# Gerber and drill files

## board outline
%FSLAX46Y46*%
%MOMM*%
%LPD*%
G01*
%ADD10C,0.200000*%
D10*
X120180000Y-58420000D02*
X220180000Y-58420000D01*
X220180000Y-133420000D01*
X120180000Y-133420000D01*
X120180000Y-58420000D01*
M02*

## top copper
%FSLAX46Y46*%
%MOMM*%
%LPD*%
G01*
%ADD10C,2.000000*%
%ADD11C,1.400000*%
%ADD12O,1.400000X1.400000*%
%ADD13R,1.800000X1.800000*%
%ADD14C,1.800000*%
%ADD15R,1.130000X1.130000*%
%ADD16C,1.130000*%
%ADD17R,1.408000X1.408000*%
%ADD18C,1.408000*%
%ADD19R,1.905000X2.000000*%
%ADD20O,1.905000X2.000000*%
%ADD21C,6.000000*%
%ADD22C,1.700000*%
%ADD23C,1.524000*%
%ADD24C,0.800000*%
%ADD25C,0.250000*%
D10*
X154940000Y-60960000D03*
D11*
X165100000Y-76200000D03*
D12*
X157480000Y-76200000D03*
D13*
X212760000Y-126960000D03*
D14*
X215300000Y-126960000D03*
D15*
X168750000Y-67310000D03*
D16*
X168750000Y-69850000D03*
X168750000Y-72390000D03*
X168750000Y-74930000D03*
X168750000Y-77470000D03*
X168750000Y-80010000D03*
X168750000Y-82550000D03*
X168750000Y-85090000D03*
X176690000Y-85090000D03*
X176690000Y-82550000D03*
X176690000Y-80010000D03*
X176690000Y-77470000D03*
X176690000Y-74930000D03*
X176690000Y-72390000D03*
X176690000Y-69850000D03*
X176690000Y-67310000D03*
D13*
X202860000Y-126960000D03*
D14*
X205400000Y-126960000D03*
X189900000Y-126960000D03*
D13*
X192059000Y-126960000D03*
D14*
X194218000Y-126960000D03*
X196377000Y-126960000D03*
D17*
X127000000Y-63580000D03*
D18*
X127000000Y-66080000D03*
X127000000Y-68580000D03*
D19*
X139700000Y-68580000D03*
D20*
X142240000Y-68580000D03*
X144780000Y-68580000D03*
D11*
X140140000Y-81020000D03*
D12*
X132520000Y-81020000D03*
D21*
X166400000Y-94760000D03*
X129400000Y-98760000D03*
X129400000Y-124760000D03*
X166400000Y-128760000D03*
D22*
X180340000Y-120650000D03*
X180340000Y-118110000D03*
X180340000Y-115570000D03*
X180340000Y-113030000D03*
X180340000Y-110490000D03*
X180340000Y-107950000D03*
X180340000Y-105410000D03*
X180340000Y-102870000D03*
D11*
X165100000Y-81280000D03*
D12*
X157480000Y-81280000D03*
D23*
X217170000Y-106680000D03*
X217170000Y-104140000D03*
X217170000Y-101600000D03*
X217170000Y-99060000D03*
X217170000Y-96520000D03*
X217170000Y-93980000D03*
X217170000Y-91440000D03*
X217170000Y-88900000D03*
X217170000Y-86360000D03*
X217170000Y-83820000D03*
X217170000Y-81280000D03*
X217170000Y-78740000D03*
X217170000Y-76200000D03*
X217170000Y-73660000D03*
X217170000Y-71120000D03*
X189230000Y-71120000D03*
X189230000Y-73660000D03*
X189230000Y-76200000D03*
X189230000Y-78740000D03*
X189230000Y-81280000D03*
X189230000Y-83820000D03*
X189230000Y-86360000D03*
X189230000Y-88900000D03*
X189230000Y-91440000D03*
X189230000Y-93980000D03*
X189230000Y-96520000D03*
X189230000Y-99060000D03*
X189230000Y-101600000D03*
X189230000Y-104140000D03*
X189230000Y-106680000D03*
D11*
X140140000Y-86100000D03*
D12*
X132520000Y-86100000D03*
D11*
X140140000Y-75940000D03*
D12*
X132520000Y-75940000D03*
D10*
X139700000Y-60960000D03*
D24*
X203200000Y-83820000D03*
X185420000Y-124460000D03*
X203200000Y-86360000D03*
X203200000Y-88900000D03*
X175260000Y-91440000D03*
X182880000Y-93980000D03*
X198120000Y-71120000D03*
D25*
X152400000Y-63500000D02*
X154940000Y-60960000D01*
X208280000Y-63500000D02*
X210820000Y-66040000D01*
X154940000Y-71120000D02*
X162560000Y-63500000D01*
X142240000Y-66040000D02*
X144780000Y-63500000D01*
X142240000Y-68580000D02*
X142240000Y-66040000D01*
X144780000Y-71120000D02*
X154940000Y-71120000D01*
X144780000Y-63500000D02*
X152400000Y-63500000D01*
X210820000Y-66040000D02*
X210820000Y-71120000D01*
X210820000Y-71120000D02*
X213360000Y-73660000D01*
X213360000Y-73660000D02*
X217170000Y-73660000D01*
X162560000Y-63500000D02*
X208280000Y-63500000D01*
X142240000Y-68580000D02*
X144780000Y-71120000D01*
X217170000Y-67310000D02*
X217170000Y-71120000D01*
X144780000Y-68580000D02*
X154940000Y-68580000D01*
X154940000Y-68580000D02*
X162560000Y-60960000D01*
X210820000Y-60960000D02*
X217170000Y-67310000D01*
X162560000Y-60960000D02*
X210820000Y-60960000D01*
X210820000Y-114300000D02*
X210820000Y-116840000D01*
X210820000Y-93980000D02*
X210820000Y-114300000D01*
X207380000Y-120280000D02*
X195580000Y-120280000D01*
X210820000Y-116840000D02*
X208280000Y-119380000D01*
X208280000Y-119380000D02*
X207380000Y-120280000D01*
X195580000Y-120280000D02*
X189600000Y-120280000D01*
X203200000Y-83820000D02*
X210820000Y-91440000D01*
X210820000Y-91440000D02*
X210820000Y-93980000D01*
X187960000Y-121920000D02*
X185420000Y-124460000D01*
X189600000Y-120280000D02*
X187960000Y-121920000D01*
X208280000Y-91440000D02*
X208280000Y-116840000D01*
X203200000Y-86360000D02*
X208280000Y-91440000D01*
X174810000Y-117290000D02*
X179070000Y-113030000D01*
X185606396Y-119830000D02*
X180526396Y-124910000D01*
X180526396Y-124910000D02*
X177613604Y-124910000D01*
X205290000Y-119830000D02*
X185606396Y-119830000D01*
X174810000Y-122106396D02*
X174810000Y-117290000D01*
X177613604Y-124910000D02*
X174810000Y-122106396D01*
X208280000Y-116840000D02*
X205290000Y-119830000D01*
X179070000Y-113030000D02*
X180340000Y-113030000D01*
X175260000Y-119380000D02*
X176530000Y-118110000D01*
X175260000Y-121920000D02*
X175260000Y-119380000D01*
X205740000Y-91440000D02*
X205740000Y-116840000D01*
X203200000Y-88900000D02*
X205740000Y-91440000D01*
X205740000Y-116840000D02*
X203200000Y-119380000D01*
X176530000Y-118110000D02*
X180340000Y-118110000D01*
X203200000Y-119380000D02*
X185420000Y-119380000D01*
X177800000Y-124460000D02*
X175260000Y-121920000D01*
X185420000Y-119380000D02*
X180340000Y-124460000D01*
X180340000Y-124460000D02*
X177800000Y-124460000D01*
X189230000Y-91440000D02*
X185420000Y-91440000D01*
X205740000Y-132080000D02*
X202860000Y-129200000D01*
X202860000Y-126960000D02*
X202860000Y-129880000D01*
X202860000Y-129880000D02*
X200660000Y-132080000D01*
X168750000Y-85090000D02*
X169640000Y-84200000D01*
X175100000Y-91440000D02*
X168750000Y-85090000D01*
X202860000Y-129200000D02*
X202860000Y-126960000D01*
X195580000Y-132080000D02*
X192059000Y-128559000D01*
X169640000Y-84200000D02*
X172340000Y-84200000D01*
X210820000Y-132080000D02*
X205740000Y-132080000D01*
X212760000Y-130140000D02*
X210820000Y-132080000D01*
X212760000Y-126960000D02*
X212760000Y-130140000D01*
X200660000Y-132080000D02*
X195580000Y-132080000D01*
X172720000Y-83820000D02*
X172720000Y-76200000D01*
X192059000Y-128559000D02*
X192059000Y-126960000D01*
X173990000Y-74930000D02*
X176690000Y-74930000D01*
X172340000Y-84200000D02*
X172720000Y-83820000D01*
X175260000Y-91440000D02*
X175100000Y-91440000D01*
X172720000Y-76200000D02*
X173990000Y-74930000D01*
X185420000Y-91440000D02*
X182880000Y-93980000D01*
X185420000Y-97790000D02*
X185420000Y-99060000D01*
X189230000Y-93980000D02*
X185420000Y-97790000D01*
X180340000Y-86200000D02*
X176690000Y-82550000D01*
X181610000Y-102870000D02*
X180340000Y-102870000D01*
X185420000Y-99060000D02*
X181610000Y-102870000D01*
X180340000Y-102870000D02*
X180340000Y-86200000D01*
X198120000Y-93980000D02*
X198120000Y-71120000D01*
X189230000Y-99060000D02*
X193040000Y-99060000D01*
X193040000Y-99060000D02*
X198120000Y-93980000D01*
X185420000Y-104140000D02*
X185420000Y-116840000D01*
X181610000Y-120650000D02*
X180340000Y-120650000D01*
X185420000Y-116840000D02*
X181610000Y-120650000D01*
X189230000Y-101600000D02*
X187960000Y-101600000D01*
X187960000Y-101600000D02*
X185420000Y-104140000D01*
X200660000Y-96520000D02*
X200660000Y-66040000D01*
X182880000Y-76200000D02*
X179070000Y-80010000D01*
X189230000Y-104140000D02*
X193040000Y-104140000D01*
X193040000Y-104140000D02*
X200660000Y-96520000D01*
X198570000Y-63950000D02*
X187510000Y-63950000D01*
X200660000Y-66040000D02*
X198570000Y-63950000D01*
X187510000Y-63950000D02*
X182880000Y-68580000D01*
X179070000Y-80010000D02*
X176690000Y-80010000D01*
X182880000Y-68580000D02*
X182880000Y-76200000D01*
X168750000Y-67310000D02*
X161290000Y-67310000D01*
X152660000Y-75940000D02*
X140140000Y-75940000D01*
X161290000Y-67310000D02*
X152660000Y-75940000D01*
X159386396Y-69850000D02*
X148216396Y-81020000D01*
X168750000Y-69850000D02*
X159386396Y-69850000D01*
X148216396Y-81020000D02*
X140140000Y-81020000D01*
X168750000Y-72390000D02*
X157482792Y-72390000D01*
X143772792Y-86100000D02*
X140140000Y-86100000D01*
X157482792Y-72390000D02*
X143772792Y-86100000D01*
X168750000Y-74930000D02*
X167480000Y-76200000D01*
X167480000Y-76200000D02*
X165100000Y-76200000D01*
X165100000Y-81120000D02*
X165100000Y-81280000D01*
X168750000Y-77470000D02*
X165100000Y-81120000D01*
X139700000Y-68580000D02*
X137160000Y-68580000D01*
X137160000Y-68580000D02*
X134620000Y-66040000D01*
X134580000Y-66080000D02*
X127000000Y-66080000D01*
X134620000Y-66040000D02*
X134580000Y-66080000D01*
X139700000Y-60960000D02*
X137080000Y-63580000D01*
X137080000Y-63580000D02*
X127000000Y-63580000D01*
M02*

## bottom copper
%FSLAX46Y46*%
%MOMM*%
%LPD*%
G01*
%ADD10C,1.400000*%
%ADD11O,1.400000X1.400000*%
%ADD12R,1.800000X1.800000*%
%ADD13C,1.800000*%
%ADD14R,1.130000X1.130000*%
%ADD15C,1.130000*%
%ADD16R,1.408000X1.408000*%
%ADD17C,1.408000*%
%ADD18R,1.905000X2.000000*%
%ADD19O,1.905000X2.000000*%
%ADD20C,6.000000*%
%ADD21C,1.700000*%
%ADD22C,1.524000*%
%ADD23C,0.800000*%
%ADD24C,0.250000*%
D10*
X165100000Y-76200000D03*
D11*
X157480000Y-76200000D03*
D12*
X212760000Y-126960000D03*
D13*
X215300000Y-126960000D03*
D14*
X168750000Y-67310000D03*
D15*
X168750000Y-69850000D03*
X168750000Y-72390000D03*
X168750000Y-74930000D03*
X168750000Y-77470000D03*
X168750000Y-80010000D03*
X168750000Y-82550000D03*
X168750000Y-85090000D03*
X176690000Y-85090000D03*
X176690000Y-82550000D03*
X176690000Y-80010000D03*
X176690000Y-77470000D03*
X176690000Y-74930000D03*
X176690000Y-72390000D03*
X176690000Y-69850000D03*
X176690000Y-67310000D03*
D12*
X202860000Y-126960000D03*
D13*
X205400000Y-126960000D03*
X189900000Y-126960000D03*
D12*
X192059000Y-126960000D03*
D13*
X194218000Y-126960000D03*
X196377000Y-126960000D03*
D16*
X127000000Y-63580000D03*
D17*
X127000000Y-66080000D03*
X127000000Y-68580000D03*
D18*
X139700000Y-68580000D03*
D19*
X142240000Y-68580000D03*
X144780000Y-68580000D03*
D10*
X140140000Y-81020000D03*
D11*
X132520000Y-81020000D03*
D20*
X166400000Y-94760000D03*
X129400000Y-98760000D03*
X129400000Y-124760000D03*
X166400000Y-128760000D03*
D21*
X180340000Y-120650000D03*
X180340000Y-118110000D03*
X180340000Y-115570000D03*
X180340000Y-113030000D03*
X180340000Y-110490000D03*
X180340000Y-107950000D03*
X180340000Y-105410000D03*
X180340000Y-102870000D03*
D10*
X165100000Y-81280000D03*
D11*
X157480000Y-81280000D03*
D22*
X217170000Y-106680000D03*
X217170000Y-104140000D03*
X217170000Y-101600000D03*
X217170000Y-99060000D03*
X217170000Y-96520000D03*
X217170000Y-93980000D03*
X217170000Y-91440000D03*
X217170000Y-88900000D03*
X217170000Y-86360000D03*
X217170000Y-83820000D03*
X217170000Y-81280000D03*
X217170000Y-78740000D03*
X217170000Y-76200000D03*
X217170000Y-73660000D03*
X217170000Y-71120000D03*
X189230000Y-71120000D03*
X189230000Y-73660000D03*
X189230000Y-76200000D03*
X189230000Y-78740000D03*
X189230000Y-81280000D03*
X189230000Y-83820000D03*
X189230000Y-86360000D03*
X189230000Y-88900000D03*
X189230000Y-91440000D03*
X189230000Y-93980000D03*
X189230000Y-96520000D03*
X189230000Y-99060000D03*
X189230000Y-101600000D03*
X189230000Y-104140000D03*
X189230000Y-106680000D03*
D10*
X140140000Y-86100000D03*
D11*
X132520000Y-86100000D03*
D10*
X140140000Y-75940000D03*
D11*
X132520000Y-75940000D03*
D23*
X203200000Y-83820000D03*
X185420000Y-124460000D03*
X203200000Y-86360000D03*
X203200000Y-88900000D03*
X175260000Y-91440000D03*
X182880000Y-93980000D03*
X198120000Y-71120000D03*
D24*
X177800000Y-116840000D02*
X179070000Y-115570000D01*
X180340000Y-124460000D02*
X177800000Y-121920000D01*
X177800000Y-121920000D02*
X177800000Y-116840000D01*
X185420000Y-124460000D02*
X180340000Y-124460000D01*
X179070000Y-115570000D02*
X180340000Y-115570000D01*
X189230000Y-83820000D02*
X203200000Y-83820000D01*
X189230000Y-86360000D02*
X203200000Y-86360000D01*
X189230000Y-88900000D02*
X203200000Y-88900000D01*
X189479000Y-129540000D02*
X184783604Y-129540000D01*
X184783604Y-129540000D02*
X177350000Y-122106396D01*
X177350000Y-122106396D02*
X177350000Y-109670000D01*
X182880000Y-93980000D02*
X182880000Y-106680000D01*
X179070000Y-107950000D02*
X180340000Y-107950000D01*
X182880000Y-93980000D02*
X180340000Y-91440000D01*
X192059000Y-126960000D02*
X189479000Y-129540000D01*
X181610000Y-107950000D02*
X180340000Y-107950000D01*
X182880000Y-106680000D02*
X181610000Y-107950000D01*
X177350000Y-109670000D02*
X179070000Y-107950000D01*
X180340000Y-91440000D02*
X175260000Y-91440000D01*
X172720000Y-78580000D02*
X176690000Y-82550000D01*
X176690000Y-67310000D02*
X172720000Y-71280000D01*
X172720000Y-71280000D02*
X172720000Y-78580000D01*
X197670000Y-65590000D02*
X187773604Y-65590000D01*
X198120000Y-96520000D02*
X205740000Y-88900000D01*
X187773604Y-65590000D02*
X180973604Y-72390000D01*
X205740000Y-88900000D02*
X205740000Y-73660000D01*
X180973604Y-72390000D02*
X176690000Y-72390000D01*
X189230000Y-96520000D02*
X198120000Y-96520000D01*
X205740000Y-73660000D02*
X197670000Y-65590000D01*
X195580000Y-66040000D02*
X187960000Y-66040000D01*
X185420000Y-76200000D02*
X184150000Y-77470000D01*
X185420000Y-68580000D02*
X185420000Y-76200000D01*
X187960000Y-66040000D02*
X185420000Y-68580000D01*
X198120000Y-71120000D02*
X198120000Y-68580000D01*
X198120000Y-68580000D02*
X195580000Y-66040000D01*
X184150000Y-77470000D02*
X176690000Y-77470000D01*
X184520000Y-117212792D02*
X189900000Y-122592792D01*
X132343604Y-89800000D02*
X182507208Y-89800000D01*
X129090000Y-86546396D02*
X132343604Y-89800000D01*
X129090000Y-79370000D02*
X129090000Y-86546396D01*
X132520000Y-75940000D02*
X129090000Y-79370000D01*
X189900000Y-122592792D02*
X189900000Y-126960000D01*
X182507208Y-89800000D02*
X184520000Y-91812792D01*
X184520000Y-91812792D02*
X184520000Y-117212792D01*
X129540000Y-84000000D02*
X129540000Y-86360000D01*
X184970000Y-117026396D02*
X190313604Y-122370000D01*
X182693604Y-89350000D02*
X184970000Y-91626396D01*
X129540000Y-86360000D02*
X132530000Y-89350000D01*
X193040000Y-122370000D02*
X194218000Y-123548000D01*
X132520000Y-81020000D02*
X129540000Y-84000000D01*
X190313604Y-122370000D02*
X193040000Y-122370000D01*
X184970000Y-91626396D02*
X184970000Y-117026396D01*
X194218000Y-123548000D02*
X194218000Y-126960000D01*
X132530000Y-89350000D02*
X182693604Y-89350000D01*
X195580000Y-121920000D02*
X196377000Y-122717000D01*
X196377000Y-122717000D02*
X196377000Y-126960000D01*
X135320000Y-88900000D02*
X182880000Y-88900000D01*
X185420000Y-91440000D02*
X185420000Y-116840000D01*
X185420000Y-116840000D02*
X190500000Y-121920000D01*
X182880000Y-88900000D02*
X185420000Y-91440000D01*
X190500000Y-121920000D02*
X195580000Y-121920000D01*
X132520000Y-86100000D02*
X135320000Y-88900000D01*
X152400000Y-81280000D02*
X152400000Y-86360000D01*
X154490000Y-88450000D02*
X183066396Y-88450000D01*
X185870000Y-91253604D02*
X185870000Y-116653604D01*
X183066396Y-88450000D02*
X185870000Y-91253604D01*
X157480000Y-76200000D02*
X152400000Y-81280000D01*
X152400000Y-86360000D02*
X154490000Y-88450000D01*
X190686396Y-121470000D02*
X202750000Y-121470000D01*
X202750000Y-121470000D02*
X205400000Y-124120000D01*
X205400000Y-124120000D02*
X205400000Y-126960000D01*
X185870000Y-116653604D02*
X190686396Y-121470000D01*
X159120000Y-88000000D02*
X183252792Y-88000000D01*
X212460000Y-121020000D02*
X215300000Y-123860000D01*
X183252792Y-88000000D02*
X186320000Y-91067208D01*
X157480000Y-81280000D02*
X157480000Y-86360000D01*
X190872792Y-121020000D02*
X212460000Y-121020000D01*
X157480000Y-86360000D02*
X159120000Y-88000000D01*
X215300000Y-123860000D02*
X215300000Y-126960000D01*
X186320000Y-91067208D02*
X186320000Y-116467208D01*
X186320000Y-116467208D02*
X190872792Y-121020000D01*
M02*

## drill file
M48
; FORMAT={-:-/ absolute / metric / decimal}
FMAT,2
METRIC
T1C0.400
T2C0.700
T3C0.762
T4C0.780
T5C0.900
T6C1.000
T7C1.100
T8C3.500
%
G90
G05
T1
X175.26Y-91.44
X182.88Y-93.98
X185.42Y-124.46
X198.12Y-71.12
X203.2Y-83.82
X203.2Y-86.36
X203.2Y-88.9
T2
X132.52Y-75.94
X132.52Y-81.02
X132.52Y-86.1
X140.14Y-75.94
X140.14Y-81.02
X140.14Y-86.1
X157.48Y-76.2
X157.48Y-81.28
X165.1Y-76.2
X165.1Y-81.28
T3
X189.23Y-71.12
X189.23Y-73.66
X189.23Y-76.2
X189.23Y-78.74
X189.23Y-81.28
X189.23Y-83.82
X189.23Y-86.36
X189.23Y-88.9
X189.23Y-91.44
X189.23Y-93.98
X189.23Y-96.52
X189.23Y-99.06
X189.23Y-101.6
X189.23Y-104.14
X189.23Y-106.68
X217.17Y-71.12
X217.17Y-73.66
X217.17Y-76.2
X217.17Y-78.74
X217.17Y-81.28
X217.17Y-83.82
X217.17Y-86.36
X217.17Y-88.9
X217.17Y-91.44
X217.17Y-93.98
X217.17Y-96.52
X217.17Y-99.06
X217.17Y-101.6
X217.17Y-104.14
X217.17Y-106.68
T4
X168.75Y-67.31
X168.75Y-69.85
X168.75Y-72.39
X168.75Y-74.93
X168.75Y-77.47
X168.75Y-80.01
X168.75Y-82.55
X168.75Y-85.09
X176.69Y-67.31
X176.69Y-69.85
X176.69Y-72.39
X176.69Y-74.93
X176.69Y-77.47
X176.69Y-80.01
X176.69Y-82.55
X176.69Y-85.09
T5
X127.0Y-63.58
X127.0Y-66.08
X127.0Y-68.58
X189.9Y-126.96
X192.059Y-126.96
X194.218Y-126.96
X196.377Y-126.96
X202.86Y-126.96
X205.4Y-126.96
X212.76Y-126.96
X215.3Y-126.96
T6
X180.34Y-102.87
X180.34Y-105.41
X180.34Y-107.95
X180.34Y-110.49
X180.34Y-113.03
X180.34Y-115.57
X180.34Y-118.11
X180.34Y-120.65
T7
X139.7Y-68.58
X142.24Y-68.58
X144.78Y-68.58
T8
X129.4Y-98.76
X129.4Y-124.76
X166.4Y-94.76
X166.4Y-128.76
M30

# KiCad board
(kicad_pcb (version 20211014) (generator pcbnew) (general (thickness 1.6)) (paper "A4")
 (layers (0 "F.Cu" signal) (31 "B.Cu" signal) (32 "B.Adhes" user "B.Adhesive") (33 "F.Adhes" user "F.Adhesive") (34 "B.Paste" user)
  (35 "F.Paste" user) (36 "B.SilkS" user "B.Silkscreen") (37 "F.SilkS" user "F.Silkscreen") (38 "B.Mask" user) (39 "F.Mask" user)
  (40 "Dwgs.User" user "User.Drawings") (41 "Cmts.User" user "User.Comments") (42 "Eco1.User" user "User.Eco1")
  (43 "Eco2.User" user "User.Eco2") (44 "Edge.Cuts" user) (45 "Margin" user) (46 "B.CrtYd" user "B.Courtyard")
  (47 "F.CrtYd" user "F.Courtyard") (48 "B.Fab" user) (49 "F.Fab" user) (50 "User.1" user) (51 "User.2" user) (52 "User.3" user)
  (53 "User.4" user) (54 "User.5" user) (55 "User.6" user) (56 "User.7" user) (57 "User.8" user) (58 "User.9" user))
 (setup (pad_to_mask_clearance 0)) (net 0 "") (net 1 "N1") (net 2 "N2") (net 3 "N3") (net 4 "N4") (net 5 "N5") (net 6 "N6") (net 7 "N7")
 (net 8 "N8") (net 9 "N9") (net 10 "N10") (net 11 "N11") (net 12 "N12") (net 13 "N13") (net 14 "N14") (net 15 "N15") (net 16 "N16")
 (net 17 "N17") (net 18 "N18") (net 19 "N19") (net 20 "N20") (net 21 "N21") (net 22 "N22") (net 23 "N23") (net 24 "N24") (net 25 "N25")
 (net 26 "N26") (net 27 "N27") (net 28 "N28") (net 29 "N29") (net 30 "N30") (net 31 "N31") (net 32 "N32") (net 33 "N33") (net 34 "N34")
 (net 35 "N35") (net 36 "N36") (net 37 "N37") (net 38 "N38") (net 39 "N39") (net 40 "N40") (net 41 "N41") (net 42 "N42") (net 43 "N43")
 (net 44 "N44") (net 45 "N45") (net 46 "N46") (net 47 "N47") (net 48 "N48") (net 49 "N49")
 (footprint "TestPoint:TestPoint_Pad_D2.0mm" (layer "F.Cu") (at 154.94 60.96)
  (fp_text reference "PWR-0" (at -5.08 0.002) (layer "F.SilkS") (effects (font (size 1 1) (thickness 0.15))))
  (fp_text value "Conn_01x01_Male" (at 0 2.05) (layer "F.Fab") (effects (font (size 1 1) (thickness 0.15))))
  (pad "1" smd circle (at 0 0) (size 2 2) (layers "F.Cu" "F.Mask") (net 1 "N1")))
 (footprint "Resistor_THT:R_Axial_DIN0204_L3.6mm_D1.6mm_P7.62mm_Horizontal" (layer "F.Cu") (at 165.1 76.2 180)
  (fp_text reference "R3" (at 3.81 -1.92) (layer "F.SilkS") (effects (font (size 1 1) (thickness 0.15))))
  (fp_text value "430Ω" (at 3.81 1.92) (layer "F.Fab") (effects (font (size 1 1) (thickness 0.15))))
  (pad "1" thru_hole circle (at 0 0 180) (size 1.4 1.4) (drill 0.7) (layers *.Cu *.Mask) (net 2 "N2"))
  (pad "2" thru_hole oval (at 7.62 0 180) (size 1.4 1.4) (drill 0.7) (layers *.Cu *.Mask) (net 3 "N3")))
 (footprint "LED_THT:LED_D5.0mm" (layer "F.Cu") (at 212.76 126.96)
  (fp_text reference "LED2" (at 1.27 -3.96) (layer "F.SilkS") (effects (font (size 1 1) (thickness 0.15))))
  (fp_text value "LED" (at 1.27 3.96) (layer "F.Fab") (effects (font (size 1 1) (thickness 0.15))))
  (pad "1" thru_hole rect (at 0 0) (size 1.8 1.8) (drill 0.9) (layers *.Cu *.Mask) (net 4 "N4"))
  (pad "2" thru_hole circle (at 2.54 0) (size 1.8 1.8) (drill 0.9) (layers *.Cu *.Mask) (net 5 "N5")))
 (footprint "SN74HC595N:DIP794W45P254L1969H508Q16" (layer "F.Cu") (at 172.72 76.2)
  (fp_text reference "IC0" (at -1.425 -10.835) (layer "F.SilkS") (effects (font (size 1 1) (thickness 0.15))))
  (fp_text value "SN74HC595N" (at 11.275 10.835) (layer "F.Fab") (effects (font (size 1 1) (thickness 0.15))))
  (pad "1" thru_hole rect locked (at -3.97 -8.89) (size 1.13 1.13) (drill 0.78) (layers *.Cu *.Mask) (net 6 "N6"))
  (pad "2" thru_hole circle locked (at -3.97 -6.35) (size 1.13 1.13) (drill 0.78) (layers *.Cu *.Mask) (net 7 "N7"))
  (pad "3" thru_hole circle locked (at -3.97 -3.81) (size 1.13 1.13) (drill 0.78) (layers *.Cu *.Mask) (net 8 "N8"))
  (pad "4" thru_hole circle locked (at -3.97 -1.27) (size 1.13 1.13) (drill 0.78) (layers *.Cu *.Mask) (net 2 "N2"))
  (pad "5" thru_hole circle locked (at -3.97 1.27) (size 1.13 1.13) (drill 0.78) (layers *.Cu *.Mask) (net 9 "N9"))
  (pad "6" thru_hole circle locked (at -3.97 3.81) (size 1.13 1.13) (drill 0.78) (layers *.Cu *.Mask) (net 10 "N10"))
  (pad "7" thru_hole circle locked (at -3.97 6.35) (size 1.13 1.13) (drill 0.78) (layers *.Cu *.Mask) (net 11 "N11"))
  (pad "8" thru_hole circle locked (at -3.97 8.89) (size 1.13 1.13) (drill 0.78) (layers *.Cu *.Mask) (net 4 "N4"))
  (pad "9" thru_hole circle locked (at 3.97 8.89) (size 1.13 1.13) (drill 0.78) (layers *.Cu *.Mask) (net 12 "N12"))
  (pad "10" thru_hole circle locked (at 3.97 6.35) (size 1.13 1.13) (drill 0.78) (layers *.Cu *.Mask) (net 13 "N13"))
  (pad "11" thru_hole circle locked (at 3.97 3.81) (size 1.13 1.13) (drill 0.78) (layers *.Cu *.Mask) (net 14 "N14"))
  (pad "12" thru_hole circle locked (at 3.97 1.27) (size 1.13 1.13) (drill 0.78) (layers *.Cu *.Mask) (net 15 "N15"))
  (pad "13" thru_hole circle locked (at 3.97 -1.27) (size 1.13 1.13) (drill 0.78) (layers *.Cu *.Mask) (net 4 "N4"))
  (pad "14" thru_hole circle locked (at 3.97 -3.81) (size 1.13 1.13) (drill 0.78) (layers *.Cu *.Mask) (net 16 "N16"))
  (pad "15" thru_hole circle locked (at 3.97 -6.35) (size 1.13 1.13) (drill 0.78) (layers *.Cu *.Mask) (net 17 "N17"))
  (pad "16" thru_hole circle locked (at 3.97 -8.89) (size 1.13 1.13) (drill 0.78) (layers *.Cu *.Mask) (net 13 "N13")))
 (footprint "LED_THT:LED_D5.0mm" (layer "F.Cu") (at 202.86 126.96)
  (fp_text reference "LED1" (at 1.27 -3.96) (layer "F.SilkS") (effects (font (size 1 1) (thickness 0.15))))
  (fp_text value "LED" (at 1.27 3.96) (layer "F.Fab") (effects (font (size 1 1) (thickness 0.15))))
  (pad "1" thru_hole rect (at 0 0) (size 1.8 1.8) (drill 0.9) (layers *.Cu *.Mask) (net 4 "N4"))
  (pad "2" thru_hole circle (at 2.54 0) (size 1.8 1.8) (drill 0.9) (layers *.Cu *.Mask) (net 3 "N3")))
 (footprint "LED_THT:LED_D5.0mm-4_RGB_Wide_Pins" (layer "F.Cu") (at 189.9 126.96)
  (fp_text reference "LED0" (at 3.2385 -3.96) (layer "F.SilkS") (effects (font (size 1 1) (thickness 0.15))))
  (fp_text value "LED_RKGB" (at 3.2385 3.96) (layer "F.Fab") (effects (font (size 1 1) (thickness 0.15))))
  (pad "1" thru_hole circle (at 0 0) (size 1.8 1.8) (drill 0.9) (layers *.Cu *.Mask) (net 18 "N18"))
  (pad "2" thru_hole rect (at 2.159 0) (size 1.8 1.8) (drill 0.9) (layers *.Cu *.Mask) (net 4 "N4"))
  (pad "3" thru_hole circle (at 4.318 0) (size 1.8 1.8) (drill 0.9) (layers *.Cu *.Mask) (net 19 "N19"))
  (pad "4" thru_hole circle (at 6.477 0) (size 1.8 1.8) (drill 0.9) (layers *.Cu *.Mask) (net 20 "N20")))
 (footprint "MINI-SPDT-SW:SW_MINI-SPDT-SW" (layer "F.Cu") (at 127 66.08 -90)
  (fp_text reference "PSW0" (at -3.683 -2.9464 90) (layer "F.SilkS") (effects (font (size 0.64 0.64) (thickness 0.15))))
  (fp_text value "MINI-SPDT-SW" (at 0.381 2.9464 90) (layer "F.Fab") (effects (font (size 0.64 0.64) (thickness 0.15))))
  (pad "1" thru_hole rect locked (at -2.5 0 270) (size 1.408 1.408) (drill 0.9) (layers *.Cu *.Mask) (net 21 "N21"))
  (pad "2" thru_hole circle locked (at 0 0 270) (size 1.408 1.408) (drill 0.9) (layers *.Cu *.Mask) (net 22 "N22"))
  (pad "3" thru_hole circle locked (at 2.5 0 270) (size 1.408 1.408) (drill 0.9) (layers *.Cu *.Mask) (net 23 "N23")))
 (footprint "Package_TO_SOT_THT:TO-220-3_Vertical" (layer "F.Cu") (at 139.7 68.58)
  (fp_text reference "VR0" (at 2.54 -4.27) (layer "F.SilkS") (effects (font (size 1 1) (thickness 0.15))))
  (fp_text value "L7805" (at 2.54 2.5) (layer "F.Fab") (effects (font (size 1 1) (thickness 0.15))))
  (pad "1" thru_hole rect (at 0 0) (size 1.905 2) (drill 1.1) (layers *.Cu *.Mask) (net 22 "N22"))
  (pad "2" thru_hole oval (at 2.54 0) (size 1.905 2) (drill 1.1) (layers *.Cu *.Mask) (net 1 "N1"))
  (pad "3" thru_hole oval (at 5.08 0) (size 1.905 2) (drill 1.1) (layers *.Cu *.Mask) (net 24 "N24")))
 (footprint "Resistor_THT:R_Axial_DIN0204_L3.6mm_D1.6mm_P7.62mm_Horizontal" (layer "F.Cu") (at 140.14 81.02 180)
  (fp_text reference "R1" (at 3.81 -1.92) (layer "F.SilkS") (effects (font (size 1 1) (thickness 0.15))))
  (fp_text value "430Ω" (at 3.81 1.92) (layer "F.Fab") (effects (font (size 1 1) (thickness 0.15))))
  (pad "1" thru_hole circle (at 0 0 180) (size 1.4 1.4) (drill 0.7) (layers *.Cu *.Mask) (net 7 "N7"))
  (pad "2" thru_hole oval (at 7.62 0 180) (size 1.4 1.4) (drill 0.7) (layers *.Cu *.Mask) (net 19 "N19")))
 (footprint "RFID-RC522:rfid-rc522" (layer "F.Cu") (at 152.4 111.76 180)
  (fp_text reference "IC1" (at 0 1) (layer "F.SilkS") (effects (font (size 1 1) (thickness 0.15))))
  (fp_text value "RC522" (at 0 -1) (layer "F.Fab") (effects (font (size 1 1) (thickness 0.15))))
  (pad "" thru_hole circle locked (at -14 17 180) (size 6 6) (drill 3.5) (layers *.Cu *.Mask))
  (pad "" thru_hole circle locked (at 23 13 180) (size 6 6) (drill 3.5) (layers *.Cu *.Mask))
  (pad "" thru_hole circle locked (at 23 -13 180) (size 6 6) (drill 3.5) (layers *.Cu *.Mask))
  (pad "" thru_hole circle locked (at -14 -17 180) (size 6 6) (drill 3.5) (layers *.Cu *.Mask))
  (pad "1" thru_hole circle locked (at -27.94 -8.89 180) (size 1.7 1.7) (drill 1) (layers *.Cu *.Mask) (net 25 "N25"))
  (pad "2" thru_hole circle locked (at -27.94 -6.35 180) (size 1.7 1.7) (drill 1) (layers *.Cu *.Mask) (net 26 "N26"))
  (pad "3" thru_hole circle locked (at -27.94 -3.81 180) (size 1.7 1.7) (drill 1) (layers *.Cu *.Mask) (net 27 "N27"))
  (pad "4" thru_hole circle locked (at -27.94 -1.27 180) (size 1.7 1.7) (drill 1) (layers *.Cu *.Mask) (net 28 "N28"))
  (pad "5" thru_hole circle locked (at -27.94 1.27 180) (size 1.7 1.7) (drill 1) (layers *.Cu *.Mask) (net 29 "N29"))
  (pad "6" thru_hole circle locked (at -27.94 3.81 180) (size 1.7 1.7) (drill 1) (layers *.Cu *.Mask) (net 4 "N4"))
  (pad "7" thru_hole circle locked (at -27.94 6.35 180) (size 1.7 1.7) (drill 1) (layers *.Cu *.Mask) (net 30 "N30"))
  (pad "8" thru_hole circle locked (at -27.94 8.89 180) (size 1.7 1.7) (drill 1) (layers *.Cu *.Mask) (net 13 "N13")))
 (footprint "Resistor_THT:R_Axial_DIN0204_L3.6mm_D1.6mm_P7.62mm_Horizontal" (layer "F.Cu") (at 165.1 81.28 180)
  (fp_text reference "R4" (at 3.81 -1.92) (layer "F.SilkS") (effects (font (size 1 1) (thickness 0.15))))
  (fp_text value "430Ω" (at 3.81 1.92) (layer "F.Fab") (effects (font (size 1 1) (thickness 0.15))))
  (pad "1" thru_hole circle (at 0 0 180) (size 1.4 1.4) (drill 0.7) (layers *.Cu *.Mask) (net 9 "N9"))
  (pad "2" thru_hole oval (at 7.62 0 180) (size 1.4 1.4) (drill 0.7) (layers *.Cu *.Mask) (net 5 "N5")))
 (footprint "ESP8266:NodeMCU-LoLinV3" (layer "F.Cu") (at 203.2 86.36 180)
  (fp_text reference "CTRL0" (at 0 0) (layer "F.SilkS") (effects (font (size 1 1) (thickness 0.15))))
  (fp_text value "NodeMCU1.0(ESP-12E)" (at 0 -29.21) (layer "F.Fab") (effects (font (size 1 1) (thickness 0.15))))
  (pad "1" thru_hole circle locked (at -13.97 -20.32 180) (size 1.524 1.524) (drill 0.762) (layers *.Cu *.Mask "F.SilkS") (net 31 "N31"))
  (pad "2" thru_hole circle locked (at -13.97 -17.78 180) (size 1.524 1.524) (drill 0.762) (layers *.Cu *.Mask "F.SilkS") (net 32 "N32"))
  (pad "3" thru_hole circle locked (at -13.97 -15.24 180) (size 1.524 1.524) (drill 0.762) (layers *.Cu *.Mask "F.SilkS") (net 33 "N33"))
  (pad "4" thru_hole circle locked (at -13.97 -12.7 180) (size 1.524 1.524) (drill 0.762) (layers *.Cu *.Mask "F.SilkS") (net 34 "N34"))
  (pad "5" thru_hole circle locked (at -13.97 -10.16 180) (size 1.524 1.524) (drill 0.762) (layers *.Cu *.Mask "F.SilkS") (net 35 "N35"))
  (pad "6" thru_hole circle locked (at -13.97 -7.62 180) (size 1.524 1.524) (drill 0.762) (layers *.Cu *.Mask "F.SilkS") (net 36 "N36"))
  (pad "7" thru_hole circle locked (at -13.97 -5.08 180) (size 1.524 1.524) (drill 0.762) (layers *.Cu *.Mask "F.SilkS") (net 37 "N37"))
  (pad "8" thru_hole circle locked (at -13.97 -2.54 180) (size 1.524 1.524) (drill 0.762) (layers *.Cu *.Mask "F.SilkS") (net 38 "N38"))
  (pad "9" thru_hole circle locked (at -13.97 0 180) (size 1.524 1.524) (drill 0.762) (layers *.Cu *.Mask "F.SilkS") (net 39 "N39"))
  (pad "10" thru_hole circle locked (at -13.97 2.54 180) (size 1.524 1.524) (drill 0.762) (layers *.Cu *.Mask "F.SilkS") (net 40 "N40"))
  (pad "11" thru_hole circle locked (at -13.97 5.08 180) (size 1.524 1.524) (drill 0.762) (layers *.Cu *.Mask "F.SilkS") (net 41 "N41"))
  (pad "12" thru_hole circle locked (at -13.97 7.62 180) (size 1.524 1.524) (drill 0.762) (layers *.Cu *.Mask "F.SilkS") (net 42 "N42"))
  (pad "13" thru_hole circle locked (at -13.97 10.16 180) (size 1.524 1.524) (drill 0.762) (layers *.Cu *.Mask "F.SilkS") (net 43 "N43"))
  (pad "14" thru_hole circle locked (at -13.97 12.7 180) (size 1.524 1.524) (drill 0.762) (layers *.Cu *.Mask "F.SilkS") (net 1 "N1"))
  (pad "15" thru_hole circle locked (at -13.97 15.24 180) (size 1.524 1.524) (drill 0.762) (layers *.Cu *.Mask "F.SilkS") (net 24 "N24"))
  (pad "16" thru_hole circle locked (at 13.97 15.24 180) (size 1.524 1.524) (drill 0.762) (layers *.Cu *.Mask "F.SilkS") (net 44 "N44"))
  (pad "17" thru_hole circle locked (at 13.97 12.7 180) (size 1.524 1.524) (drill 0.762) (layers *.Cu *.Mask "F.SilkS") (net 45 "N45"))
  (pad "18" thru_hole circle locked (at 13.97 10.16 180) (size 1.524 1.524) (drill 0.762) (layers *.Cu *.Mask "F.SilkS") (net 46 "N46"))
  (pad "19" thru_hole circle locked (at 13.97 7.62 180) (size 1.524 1.524) (drill 0.762) (layers *.Cu *.Mask "F.SilkS") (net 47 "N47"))
  (pad "20" thru_hole circle locked (at 13.97 5.08 180) (size 1.524 1.524) (drill 0.762) (layers *.Cu *.Mask "F.SilkS") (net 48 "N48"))
  (pad "21" thru_hole circle locked (at 13.97 2.54 180) (size 1.524 1.524) (drill 0.762) (layers *.Cu *.Mask "F.SilkS") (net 27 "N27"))
  (pad "22" thru_hole circle locked (at 13.97 0 180) (size 1.524 1.524) (drill 0.762) (layers *.Cu *.Mask "F.SilkS") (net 28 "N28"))
  (pad "23" thru_hole circle locked (at 13.97 -2.54 180) (size 1.524 1.524) (drill 0.762) (layers *.Cu *.Mask "F.SilkS") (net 26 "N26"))
  (pad "24" thru_hole circle locked (at 13.97 -5.08 180) (size 1.524 1.524) (drill 0.762) (layers *.Cu *.Mask "F.SilkS") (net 4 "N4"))
  (pad "25" thru_hole circle locked (at 13.97 -7.62 180) (size 1.524 1.524) (drill 0.762) (layers *.Cu *.Mask "F.SilkS") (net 13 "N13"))
  (pad "26" thru_hole circle locked (at 13.97 -10.16 180) (size 1.524 1.524) (drill 0.762) (layers *.Cu *.Mask "F.SilkS") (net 16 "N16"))
  (pad "27" thru_hole circle locked (at 13.97 -12.7 180) (size 1.524 1.524) (drill 0.762) (layers *.Cu *.Mask "F.SilkS") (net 15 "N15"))
  (pad "28" thru_hole circle locked (at 13.97 -15.24 180) (size 1.524 1.524) (drill 0.762) (layers *.Cu *.Mask "F.SilkS") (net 25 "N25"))
  (pad "29" thru_hole circle locked (at 13.97 -17.78 180) (size 1.524 1.524) (drill 0.762) (layers *.Cu *.Mask "F.SilkS") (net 14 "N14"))
  (pad "30" thru_hole circle locked (at 13.97 -20.32 180) (size 1.524 1.524) (drill 0.762) (layers *.Cu *.Mask "F.SilkS") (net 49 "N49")))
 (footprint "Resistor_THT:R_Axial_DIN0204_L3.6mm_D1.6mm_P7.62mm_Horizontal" (layer "F.Cu") (at 140.14 86.1 180)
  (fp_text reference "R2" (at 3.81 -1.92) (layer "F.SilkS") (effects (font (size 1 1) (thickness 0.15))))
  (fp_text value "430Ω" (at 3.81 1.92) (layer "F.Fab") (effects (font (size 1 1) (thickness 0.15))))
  (pad "1" thru_hole circle (at 0 0 180) (size 1.4 1.4) (drill 0.7) (layers *.Cu *.Mask) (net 8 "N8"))
  (pad "2" thru_hole oval (at 7.62 0 180) (size 1.4 1.4) (drill 0.7) (layers *.Cu *.Mask) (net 20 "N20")))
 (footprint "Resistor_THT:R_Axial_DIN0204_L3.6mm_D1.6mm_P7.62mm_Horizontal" (layer "F.Cu") (at 140.14 75.94 180)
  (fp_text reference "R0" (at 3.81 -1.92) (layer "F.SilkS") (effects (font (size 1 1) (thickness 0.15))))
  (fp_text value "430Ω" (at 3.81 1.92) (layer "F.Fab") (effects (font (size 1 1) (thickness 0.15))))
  (pad "1" thru_hole circle (at 0 0 180) (size 1.4 1.4) (drill 0.7) (layers *.Cu *.Mask) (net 6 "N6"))
  (pad "2" thru_hole oval (at 7.62 0 180) (size 1.4 1.4) (drill 0.7) (layers *.Cu *.Mask) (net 18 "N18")))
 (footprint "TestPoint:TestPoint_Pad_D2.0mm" (layer "F.Cu") (at 139.7 60.96)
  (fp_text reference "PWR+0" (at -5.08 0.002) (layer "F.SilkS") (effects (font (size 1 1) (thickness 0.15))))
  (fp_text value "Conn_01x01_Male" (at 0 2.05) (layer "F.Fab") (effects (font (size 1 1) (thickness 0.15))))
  (pad "1" smd circle (at 0 0) (size 2 2) (layers "F.Cu" "F.Mask") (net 21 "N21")))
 (gr_rect (start 120.18 58.42) (end 220.18 133.42) (layer "Edge.Cuts") (width 0.2) (fill none))
 (segment (start 152.4 63.5) (end 154.94 60.96) (width 0.25) (layer "F.Cu") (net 1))
 (segment (start 208.28 63.5) (end 210.82 66.04) (width 0.25) (layer "F.Cu") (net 1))
 (segment (start 154.94 71.12) (end 162.56 63.5) (width 0.25) (layer "F.Cu") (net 1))
 (segment (start 142.24 66.04) (end 144.78 63.5) (width 0.25) (layer "F.Cu") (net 1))
 (segment (start 142.24 68.58) (end 142.24 66.04) (width 0.25) (layer "F.Cu") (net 1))
 (segment (start 144.78 71.12) (end 154.94 71.12) (width 0.25) (layer "F.Cu") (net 1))
 (segment (start 144.78 63.5) (end 152.4 63.5) (width 0.25) (layer "F.Cu") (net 1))
 (segment (start 210.82 66.04) (end 210.82 71.12) (width 0.25) (layer "F.Cu") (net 1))
 (segment (start 210.82 71.12) (end 213.36 73.66) (width 0.25) (layer "F.Cu") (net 1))
 (segment (start 213.36 73.66) (end 217.17 73.66) (width 0.25) (layer "F.Cu") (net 1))
 (segment (start 162.56 63.5) (end 208.28 63.5) (width 0.25) (layer "F.Cu") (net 1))
 (segment (start 142.24 68.58) (end 144.78 71.12) (width 0.25) (layer "F.Cu") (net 1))
 (segment (start 217.17 67.31) (end 217.17 71.12) (width 0.25) (layer "F.Cu") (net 24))
 (segment (start 144.78 68.58) (end 154.94 68.58) (width 0.25) (layer "F.Cu") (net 24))
 (segment (start 154.94 68.58) (end 162.56 60.96) (width 0.25) (layer "F.Cu") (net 24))
 (segment (start 210.82 60.96) (end 217.17 67.31) (width 0.25) (layer "F.Cu") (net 24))
 (segment (start 162.56 60.96) (end 210.82 60.96) (width 0.25) (layer "F.Cu") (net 24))
 (segment (start 210.82 114.3) (end 210.82 116.84) (width 0.25) (layer "F.Cu") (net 27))
 (segment (start 210.82 93.98) (end 210.82 114.3) (width 0.25) (layer "F.Cu") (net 27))
 (segment (start 207.38 120.28) (end 195.58 120.28) (width 0.25) (layer "F.Cu") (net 27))
 (segment (start 210.82 116.84) (end 208.28 119.38) (width 0.25) (layer "F.Cu") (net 27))
 (segment (start 208.28 119.38) (end 207.38 120.28) (width 0.25) (layer "F.Cu") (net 27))
 (segment (start 195.58 120.28) (end 189.6 120.28) (width 0.25) (layer "F.Cu") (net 27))
 (segment (start 203.2 83.82) (end 210.82 91.44) (width 0.25) (layer "F.Cu") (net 27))
 (segment (start 210.82 91.44) (end 210.82 93.98) (width 0.25) (layer "F.Cu") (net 27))
 (segment (start 187.96 121.92) (end 185.42 124.46) (width 0.25) (layer "F.Cu") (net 27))
 (segment (start 189.6 120.28) (end 187.96 121.92) (width 0.25) (layer "F.Cu") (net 27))
 (via (at 203.2 83.82) (size 0.8) (drill 0.4) (layers "F.Cu" "B.Cu") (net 27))
 (via (at 185.42 124.46) (size 0.8) (drill 0.4) (layers "F.Cu" "B.Cu") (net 27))
 (segment (start 177.8 116.84) (end 179.07 115.57) (width 0.25) (layer "B.Cu") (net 27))
 (segment (start 180.34 124.46) (end 177.8 121.92) (width 0.25) (layer "B.Cu") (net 27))
 (segment (start 177.8 121.92) (end 177.8 116.84) (width 0.25) (layer "B.Cu") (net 27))
 (segment (start 185.42 124.46) (end 180.34 124.46) (width 0.25) (layer "B.Cu") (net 27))
 (segment (start 179.07 115.57) (end 180.34 115.57) (width 0.25) (layer "B.Cu") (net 27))
 (segment (start 189.23 83.82) (end 203.2 83.82) (width 0.25) (layer "B.Cu") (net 27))
 (segment (start 208.28 91.44) (end 208.28 116.84) (width 0.25) (layer "F.Cu") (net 28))
 (segment (start 203.2 86.36) (end 208.28 91.44) (width 0.25) (layer "F.Cu") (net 28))
 (segment (start 174.81 117.29) (end 179.07 113.03) (width 0.25) (layer "F.Cu") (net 28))
 (segment (start 185.606396 119.83) (end 180.526396 124.91) (width 0.25) (layer "F.Cu") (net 28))
 (segment (start 180.526396 124.91) (end 177.613604 124.91) (width 0.25) (layer "F.Cu") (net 28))
 (segment (start 205.29 119.83) (end 185.606396 119.83) (width 0.25) (layer "F.Cu") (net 28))
 (segment (start 174.81 122.106396) (end 174.81 117.29) (width 0.25) (layer "F.Cu") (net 28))
 (segment (start 177.613604 124.91) (end 174.81 122.106396) (width 0.25) (layer "F.Cu") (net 28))
 (segment (start 208.28 116.84) (end 205.29 119.83) (width 0.25) (layer "F.Cu") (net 28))
 (segment (start 179.07 113.03) (end 180.34 113.03) (width 0.25) (layer "F.Cu") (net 28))
 (via (at 203.2 86.36) (size 0.8) (drill 0.4) (layers "F.Cu" "B.Cu") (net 28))
 (segment (start 189.23 86.36) (end 203.2 86.36) (width 0.25) (layer "B.Cu") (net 28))
 (segment (start 175.26 119.38) (end 176.53 118.11) (width 0.25) (layer "F.Cu") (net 26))
 (segment (start 175.26 121.92) (end 175.26 119.38) (width 0.25) (layer "F.Cu") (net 26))
 (segment (start 205.74 91.44) (end 205.74 116.84) (width 0.25) (layer "F.Cu") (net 26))
 (segment (start 203.2 88.9) (end 205.74 91.44) (width 0.25) (layer "F.Cu") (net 26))
 (segment (start 205.74 116.84) (end 203.2 119.38) (width 0.25) (layer "F.Cu") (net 26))
 (segment (start 176.53 118.11) (end 180.34 118.11) (width 0.25) (layer "F.Cu") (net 26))
 (segment (start 203.2 119.38) (end 185.42 119.38) (width 0.25) (layer "F.Cu") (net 26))
 (segment (start 177.8 124.46) (end 175.26 121.92) (width 0.25) (layer "F.Cu") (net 26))
 (segment (start 185.42 119.38) (end 180.34 124.46) (width 0.25) (layer "F.Cu") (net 26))
 (segment (start 180.34 124.46) (end 177.8 124.46) (width 0.25) (layer "F.Cu") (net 26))
 (via (at 203.2 88.9) (size 0.8) (drill 0.4) (layers "F.Cu" "B.Cu") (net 26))
 (segment (start 189.23 88.9) (end 203.2 88.9) (width 0.25) (layer "B.Cu") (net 26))
 (segment (start 189.23 91.44) (end 185.42 91.44) (width 0.25) (layer "F.Cu") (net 4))
 (segment (start 205.74 132.08) (end 202.86 129.2) (width 0.25) (layer "F.Cu") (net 4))
 (segment (start 202.86 126.96) (end 202.86 129.88) (width 0.25) (layer "F.Cu") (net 4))
 (segment (start 202.86 129.88) (end 200.66 132.08) (width 0.25) (layer "F.Cu") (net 4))
 (segment (start 168.75 85.09) (end 169.64 84.2) (width 0.25) (layer "F.Cu") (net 4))
 (segment (start 175.1 91.44) (end 168.75 85.09) (width 0.25) (layer "F.Cu") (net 4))
 (segment (start 202.86 129.2) (end 202.86 126.96) (width 0.25) (layer "F.Cu") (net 4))
 (segment (start 195.58 132.08) (end 192.059 128.559) (width 0.25) (layer "F.Cu") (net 4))
 (segment (start 169.64 84.2) (end 172.34 84.2) (width 0.25) (layer "F.Cu") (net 4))
 (segment (start 210.82 132.08) (end 205.74 132.08) (width 0.25) (layer "F.Cu") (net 4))
 (segment (start 212.76 130.14) (end 210.82 132.08) (width 0.25) (layer "F.Cu") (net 4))
 (segment (start 212.76 126.96) (end 212.76 130.14) (width 0.25) (layer "F.Cu") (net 4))
 (segment (start 200.66 132.08) (end 195.58 132.08) (width 0.25) (layer "F.Cu") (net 4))
 (segment (start 172.72 83.82) (end 172.72 76.2) (width 0.25) (layer "F.Cu") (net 4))
 (segment (start 192.059 128.559) (end 192.059 126.96) (width 0.25) (layer "F.Cu") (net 4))
 (segment (start 173.99 74.93) (end 176.69 74.93) (width 0.25) (layer "F.Cu") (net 4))
 (segment (start 172.34 84.2) (end 172.72 83.82) (width 0.25) (layer "F.Cu") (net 4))
 (segment (start 175.26 91.44) (end 175.1 91.44) (width 0.25) (layer "F.Cu") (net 4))
 (segment (start 172.72 76.2) (end 173.99 74.93) (width 0.25) (layer "F.Cu") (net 4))
 (segment (start 185.42 91.44) (end 182.88 93.98) (width 0.25) (layer "F.Cu") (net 4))
 (via (at 175.26 91.44) (size 0.8) (drill 0.4) (layers "F.Cu" "B.Cu") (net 4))
 (via (at 182.88 93.98) (size 0.8) (drill 0.4) (layers "F.Cu" "B.Cu") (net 4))
 (segment (start 189.479 129.54) (end 184.783604 129.54) (width 0.25) (layer "B.Cu") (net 4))
 (segment (start 184.783604 129.54) (end 177.35 122.106396) (width 0.25) (layer "B.Cu") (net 4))
 (segment (start 177.35 122.106396) (end 177.35 109.67) (width 0.25) (layer "B.Cu") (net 4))
 (segment (start 182.88 93.98) (end 182.88 106.68) (width 0.25) (layer "B.Cu") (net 4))
 (segment (start 179.07 107.95) (end 180.34 107.95) (width 0.25) (layer "B.Cu") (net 4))
 (segment (start 182.88 93.98) (end 180.34 91.44) (width 0.25) (layer "B.Cu") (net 4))
 (segment (start 192.059 126.96) (end 189.479 129.54) (width 0.25) (layer "B.Cu") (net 4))
 (segment (start 181.61 107.95) (end 180.34 107.95) (width 0.25) (layer "B.Cu") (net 4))
 (segment (start 182.88 106.68) (end 181.61 107.95) (width 0.25) (layer "B.Cu") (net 4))
 (segment (start 177.35 109.67) (end 179.07 107.95) (width 0.25) (layer "B.Cu") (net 4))
 (segment (start 180.34 91.44) (end 175.26 91.44) (width 0.25) (layer "B.Cu") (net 4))
 (segment (start 185.42 97.79) (end 185.42 99.06) (width 0.25) (layer "F.Cu") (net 13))
 (segment (start 189.23 93.98) (end 185.42 97.79) (width 0.25) (layer "F.Cu") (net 13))
 (segment (start 180.34 86.2) (end 176.69 82.55) (width 0.25) (layer "F.Cu") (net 13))
 (segment (start 181.61 102.87) (end 180.34 102.87) (width 0.25) (layer "F.Cu") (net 13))
 (segment (start 185.42 99.06) (end 181.61 102.87) (width 0.25) (layer "F.Cu") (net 13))
 (segment (start 180.34 102.87) (end 180.34 86.2) (width 0.25) (layer "F.Cu") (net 13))
 (segment (start 172.72 78.58) (end 176.69 82.55) (width 0.25) (layer "B.Cu") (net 13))
 (segment (start 176.69 67.31) (end 172.72 71.28) (width 0.25) (layer "B.Cu") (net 13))
 (segment (start 172.72 71.28) (end 172.72 78.58) (width 0.25) (layer "B.Cu") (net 13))
 (segment (start 197.67 65.59) (end 187.773604 65.59) (width 0.25) (layer "B.Cu") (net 16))
 (segment (start 198.12 96.52) (end 205.74 88.9) (width 0.25) (layer "B.Cu") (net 16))
 (segment (start 187.773604 65.59) (end 180.973604 72.39) (width 0.25) (layer "B.Cu") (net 16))
 (segment (start 205.74 88.9) (end 205.74 73.66) (width 0.25) (layer "B.Cu") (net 16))
 (segment (start 180.973604 72.39) (end 176.69 72.39) (width 0.25) (layer "B.Cu") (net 16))
 (segment (start 189.23 96.52) (end 198.12 96.52) (width 0.25) (layer "B.Cu") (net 16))
 (segment (start 205.74 73.66) (end 197.67 65.59) (width 0.25) (layer "B.Cu") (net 16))
 (segment (start 198.12 93.98) (end 198.12 71.12) (width 0.25) (layer "F.Cu") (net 15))
 (segment (start 189.23 99.06) (end 193.04 99.06) (width 0.25) (layer "F.Cu") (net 15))
 (segment (start 193.04 99.06) (end 198.12 93.98) (width 0.25) (layer "F.Cu") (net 15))
 (via (at 198.12 71.12) (size 0.8) (drill 0.4) (layers "F.Cu" "B.Cu") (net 15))
 (segment (start 195.58 66.04) (end 187.96 66.04) (width 0.25) (layer "B.Cu") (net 15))
 (segment (start 185.42 76.2) (end 184.15 77.47) (width 0.25) (layer "B.Cu") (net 15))
 (segment (start 185.42 68.58) (end 185.42 76.2) (width 0.25) (layer "B.Cu") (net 15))
 (segment (start 187.96 66.04) (end 185.42 68.58) (width 0.25) (layer "B.Cu") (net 15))
 (segment (start 198.12 71.12) (end 198.12 68.58) (width 0.25) (layer "B.Cu") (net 15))
 (segment (start 198.12 68.58) (end 195.58 66.04) (width 0.25) (layer "B.Cu") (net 15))
 (segment (start 184.15 77.47) (end 176.69 77.47) (width 0.25) (layer "B.Cu") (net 15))
 (segment (start 185.42 104.14) (end 185.42 116.84) (width 0.25) (layer "F.Cu") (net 25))
 (segment (start 181.61 120.65) (end 180.34 120.65) (width 0.25) (layer "F.Cu") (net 25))
 (segment (start 185.42 116.84) (end 181.61 120.65) (width 0.25) (layer "F.Cu") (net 25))
 (segment (start 189.23 101.6) (end 187.96 101.6) (width 0.25) (layer "F.Cu") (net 25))
 (segment (start 187.96 101.6) (end 185.42 104.14) (width 0.25) (layer "F.Cu") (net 25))
 (segment (start 200.66 96.52) (end 200.66 66.04) (width 0.25) (layer "F.Cu") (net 14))
 (segment (start 182.88 76.2) (end 179.07 80.01) (width 0.25) (layer "F.Cu") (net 14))
 (segment (start 189.23 104.14) (end 193.04 104.14) (width 0.25) (layer "F.Cu") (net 14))
 (segment (start 193.04 104.14) (end 200.66 96.52) (width 0.25) (layer "F.Cu") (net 14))
 (segment (start 198.57 63.95) (end 187.51 63.95) (width 0.25) (layer "F.Cu") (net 14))
 (segment (start 200.66 66.04) (end 198.57 63.95) (width 0.25) (layer "F.Cu") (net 14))
 (segment (start 187.51 63.95) (end 182.88 68.58) (width 0.25) (layer "F.Cu") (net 14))
 (segment (start 179.07 80.01) (end 176.69 80.01) (width 0.25) (layer "F.Cu") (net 14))
 (segment (start 182.88 68.58) (end 182.88 76.2) (width 0.25) (layer "F.Cu") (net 14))
 (segment (start 168.75 67.31) (end 161.29 67.31) (width 0.25) (layer "F.Cu") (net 6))
 (segment (start 152.66 75.94) (end 140.14 75.94) (width 0.25) (layer "F.Cu") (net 6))
 (segment (start 161.29 67.31) (end 152.66 75.94) (width 0.25) (layer "F.Cu") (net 6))
 (segment (start 159.386396 69.85) (end 148.216396 81.02) (width 0.25) (layer "F.Cu") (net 7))
 (segment (start 168.75 69.85) (end 159.386396 69.85) (width 0.25) (layer "F.Cu") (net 7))
 (segment (start 148.216396 81.02) (end 140.14 81.02) (width 0.25) (layer "F.Cu") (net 7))
 (segment (start 168.75 72.39) (end 157.482792 72.39) (width 0.25) (layer "F.Cu") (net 8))
 (segment (start 143.772792 86.1) (end 140.14 86.1) (width 0.25) (layer "F.Cu") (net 8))
 (segment (start 157.482792 72.39) (end 143.772792 86.1) (width 0.25) (layer "F.Cu") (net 8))
 (segment (start 168.75 74.93) (end 167.48 76.2) (width 0.25) (layer "F.Cu") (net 2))
 (segment (start 167.48 76.2) (end 165.1 76.2) (width 0.25) (layer "F.Cu") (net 2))
 (segment (start 165.1 81.12) (end 165.1 81.28) (width 0.25) (layer "F.Cu") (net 9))
 (segment (start 168.75 77.47) (end 165.1 81.12) (width 0.25) (layer "F.Cu") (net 9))
 (segment (start 184.52 117.212792) (end 189.9 122.592792) (width 0.25) (layer "B.Cu") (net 18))
 (segment (start 132.343604 89.8) (end 182.507208 89.8) (width 0.25) (layer "B.Cu") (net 18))
 (segment (start 129.09 86.546396) (end 132.343604 89.8) (width 0.25) (layer "B.Cu") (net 18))
 (segment (start 129.09 79.37) (end 129.09 86.546396) (width 0.25) (layer "B.Cu") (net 18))
 (segment (start 132.52 75.94) (end 129.09 79.37) (width 0.25) (layer "B.Cu") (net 18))
 (segment (start 189.9 122.592792) (end 189.9 126.96) (width 0.25) (layer "B.Cu") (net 18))
 (segment (start 182.507208 89.8) (end 184.52 91.812792) (width 0.25) (layer "B.Cu") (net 18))
 (segment (start 184.52 91.812792) (end 184.52 117.212792) (width 0.25) (layer "B.Cu") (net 18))
 (segment (start 129.54 84) (end 129.54 86.36) (width 0.25) (layer "B.Cu") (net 19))
 (segment (start 184.97 117.026396) (end 190.313604 122.37) (width 0.25) (layer "B.Cu") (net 19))
 (segment (start 182.693604 89.35) (end 184.97 91.626396) (width 0.25) (layer "B.Cu") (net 19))
 (segment (start 129.54 86.36) (end 132.53 89.35) (width 0.25) (layer "B.Cu") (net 19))
 (segment (start 193.04 122.37) (end 194.218 123.548) (width 0.25) (layer "B.Cu") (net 19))
 (segment (start 132.52 81.02) (end 129.54 84) (width 0.25) (layer "B.Cu") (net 19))
 (segment (start 190.313604 122.37) (end 193.04 122.37) (width 0.25) (layer "B.Cu") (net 19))
 (segment (start 184.97 91.626396) (end 184.97 117.026396) (width 0.25) (layer "B.Cu") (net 19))
 (segment (start 194.218 123.548) (end 194.218 126.96) (width 0.25) (layer "B.Cu") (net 19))
 (segment (start 132.53 89.35) (end 182.693604 89.35) (width 0.25) (layer "B.Cu") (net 19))
 (segment (start 195.58 121.92) (end 196.377 122.717) (width 0.25) (layer "B.Cu") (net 20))
 (segment (start 196.377 122.717) (end 196.377 126.96) (width 0.25) (layer "B.Cu") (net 20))
 (segment (start 135.32 88.9) (end 182.88 88.9) (width 0.25) (layer "B.Cu") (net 20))
 (segment (start 185.42 91.44) (end 185.42 116.84) (width 0.25) (layer "B.Cu") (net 20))
 (segment (start 185.42 116.84) (end 190.5 121.92) (width 0.25) (layer "B.Cu") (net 20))
 (segment (start 182.88 88.9) (end 185.42 91.44) (width 0.25) (layer "B.Cu") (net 20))
 (segment (start 190.5 121.92) (end 195.58 121.92) (width 0.25) (layer "B.Cu") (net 20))
 (segment (start 132.52 86.1) (end 135.32 88.9) (width 0.25) (layer "B.Cu") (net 20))
 (segment (start 152.4 81.28) (end 152.4 86.36) (width 0.25) (layer "B.Cu") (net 3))
 (segment (start 154.49 88.45) (end 183.066396 88.45) (width 0.25) (layer "B.Cu") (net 3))
 (segment (start 185.87 91.253604) (end 185.87 116.653604) (width 0.25) (layer "B.Cu") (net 3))
 (segment (start 183.066396 88.45) (end 185.87 91.253604) (width 0.25) (layer "B.Cu") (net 3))
 (segment (start 157.48 76.2) (end 152.4 81.28) (width 0.25) (layer "B.Cu") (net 3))
 (segment (start 152.4 86.36) (end 154.49 88.45) (width 0.25) (layer "B.Cu") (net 3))
 (segment (start 190.686396 121.47) (end 202.75 121.47) (width 0.25) (layer "B.Cu") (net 3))
 (segment (start 202.75 121.47) (end 205.4 124.12) (width 0.25) (layer "B.Cu") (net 3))
 (segment (start 205.4 124.12) (end 205.4 126.96) (width 0.25) (layer "B.Cu") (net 3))
 (segment (start 185.87 116.653604) (end 190.686396 121.47) (width 0.25) (layer "B.Cu") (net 3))
 (segment (start 159.12 88) (end 183.252792 88) (width 0.25) (layer "B.Cu") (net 5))
 (segment (start 212.46 121.02) (end 215.3 123.86) (width 0.25) (layer "B.Cu") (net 5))
 (segment (start 183.252792 88) (end 186.32 91.067208) (width 0.25) (layer "B.Cu") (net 5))
 (segment (start 157.48 81.28) (end 157.48 86.36) (width 0.25) (layer "B.Cu") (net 5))
 (segment (start 190.872792 121.02) (end 212.46 121.02) (width 0.25) (layer "B.Cu") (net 5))
 (segment (start 157.48 86.36) (end 159.12 88) (width 0.25) (layer "B.Cu") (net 5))
 (segment (start 215.3 123.86) (end 215.3 126.96) (width 0.25) (layer "B.Cu") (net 5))
 (segment (start 186.32 91.067208) (end 186.32 116.467208) (width 0.25) (layer "B.Cu") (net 5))
 (segment (start 186.32 116.467208) (end 190.872792 121.02) (width 0.25) (layer "B.Cu") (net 5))
 (segment (start 139.7 68.58) (end 137.16 68.58) (width 0.25) (layer "F.Cu") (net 22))
 (segment (start 137.16 68.58) (end 134.62 66.04) (width 0.25) (layer "F.Cu") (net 22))
 (segment (start 134.58 66.08) (end 127 66.08) (width 0.25) (layer "F.Cu") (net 22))
 (segment (start 134.62 66.04) (end 134.58 66.08) (width 0.25) (layer "F.Cu") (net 22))
 (segment (start 139.7 60.96) (end 137.08 63.58) (width 0.25) (layer "F.Cu") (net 21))
 (segment (start 137.08 63.58) (end 127 63.58) (width 0.25) (layer "F.Cu") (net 21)))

